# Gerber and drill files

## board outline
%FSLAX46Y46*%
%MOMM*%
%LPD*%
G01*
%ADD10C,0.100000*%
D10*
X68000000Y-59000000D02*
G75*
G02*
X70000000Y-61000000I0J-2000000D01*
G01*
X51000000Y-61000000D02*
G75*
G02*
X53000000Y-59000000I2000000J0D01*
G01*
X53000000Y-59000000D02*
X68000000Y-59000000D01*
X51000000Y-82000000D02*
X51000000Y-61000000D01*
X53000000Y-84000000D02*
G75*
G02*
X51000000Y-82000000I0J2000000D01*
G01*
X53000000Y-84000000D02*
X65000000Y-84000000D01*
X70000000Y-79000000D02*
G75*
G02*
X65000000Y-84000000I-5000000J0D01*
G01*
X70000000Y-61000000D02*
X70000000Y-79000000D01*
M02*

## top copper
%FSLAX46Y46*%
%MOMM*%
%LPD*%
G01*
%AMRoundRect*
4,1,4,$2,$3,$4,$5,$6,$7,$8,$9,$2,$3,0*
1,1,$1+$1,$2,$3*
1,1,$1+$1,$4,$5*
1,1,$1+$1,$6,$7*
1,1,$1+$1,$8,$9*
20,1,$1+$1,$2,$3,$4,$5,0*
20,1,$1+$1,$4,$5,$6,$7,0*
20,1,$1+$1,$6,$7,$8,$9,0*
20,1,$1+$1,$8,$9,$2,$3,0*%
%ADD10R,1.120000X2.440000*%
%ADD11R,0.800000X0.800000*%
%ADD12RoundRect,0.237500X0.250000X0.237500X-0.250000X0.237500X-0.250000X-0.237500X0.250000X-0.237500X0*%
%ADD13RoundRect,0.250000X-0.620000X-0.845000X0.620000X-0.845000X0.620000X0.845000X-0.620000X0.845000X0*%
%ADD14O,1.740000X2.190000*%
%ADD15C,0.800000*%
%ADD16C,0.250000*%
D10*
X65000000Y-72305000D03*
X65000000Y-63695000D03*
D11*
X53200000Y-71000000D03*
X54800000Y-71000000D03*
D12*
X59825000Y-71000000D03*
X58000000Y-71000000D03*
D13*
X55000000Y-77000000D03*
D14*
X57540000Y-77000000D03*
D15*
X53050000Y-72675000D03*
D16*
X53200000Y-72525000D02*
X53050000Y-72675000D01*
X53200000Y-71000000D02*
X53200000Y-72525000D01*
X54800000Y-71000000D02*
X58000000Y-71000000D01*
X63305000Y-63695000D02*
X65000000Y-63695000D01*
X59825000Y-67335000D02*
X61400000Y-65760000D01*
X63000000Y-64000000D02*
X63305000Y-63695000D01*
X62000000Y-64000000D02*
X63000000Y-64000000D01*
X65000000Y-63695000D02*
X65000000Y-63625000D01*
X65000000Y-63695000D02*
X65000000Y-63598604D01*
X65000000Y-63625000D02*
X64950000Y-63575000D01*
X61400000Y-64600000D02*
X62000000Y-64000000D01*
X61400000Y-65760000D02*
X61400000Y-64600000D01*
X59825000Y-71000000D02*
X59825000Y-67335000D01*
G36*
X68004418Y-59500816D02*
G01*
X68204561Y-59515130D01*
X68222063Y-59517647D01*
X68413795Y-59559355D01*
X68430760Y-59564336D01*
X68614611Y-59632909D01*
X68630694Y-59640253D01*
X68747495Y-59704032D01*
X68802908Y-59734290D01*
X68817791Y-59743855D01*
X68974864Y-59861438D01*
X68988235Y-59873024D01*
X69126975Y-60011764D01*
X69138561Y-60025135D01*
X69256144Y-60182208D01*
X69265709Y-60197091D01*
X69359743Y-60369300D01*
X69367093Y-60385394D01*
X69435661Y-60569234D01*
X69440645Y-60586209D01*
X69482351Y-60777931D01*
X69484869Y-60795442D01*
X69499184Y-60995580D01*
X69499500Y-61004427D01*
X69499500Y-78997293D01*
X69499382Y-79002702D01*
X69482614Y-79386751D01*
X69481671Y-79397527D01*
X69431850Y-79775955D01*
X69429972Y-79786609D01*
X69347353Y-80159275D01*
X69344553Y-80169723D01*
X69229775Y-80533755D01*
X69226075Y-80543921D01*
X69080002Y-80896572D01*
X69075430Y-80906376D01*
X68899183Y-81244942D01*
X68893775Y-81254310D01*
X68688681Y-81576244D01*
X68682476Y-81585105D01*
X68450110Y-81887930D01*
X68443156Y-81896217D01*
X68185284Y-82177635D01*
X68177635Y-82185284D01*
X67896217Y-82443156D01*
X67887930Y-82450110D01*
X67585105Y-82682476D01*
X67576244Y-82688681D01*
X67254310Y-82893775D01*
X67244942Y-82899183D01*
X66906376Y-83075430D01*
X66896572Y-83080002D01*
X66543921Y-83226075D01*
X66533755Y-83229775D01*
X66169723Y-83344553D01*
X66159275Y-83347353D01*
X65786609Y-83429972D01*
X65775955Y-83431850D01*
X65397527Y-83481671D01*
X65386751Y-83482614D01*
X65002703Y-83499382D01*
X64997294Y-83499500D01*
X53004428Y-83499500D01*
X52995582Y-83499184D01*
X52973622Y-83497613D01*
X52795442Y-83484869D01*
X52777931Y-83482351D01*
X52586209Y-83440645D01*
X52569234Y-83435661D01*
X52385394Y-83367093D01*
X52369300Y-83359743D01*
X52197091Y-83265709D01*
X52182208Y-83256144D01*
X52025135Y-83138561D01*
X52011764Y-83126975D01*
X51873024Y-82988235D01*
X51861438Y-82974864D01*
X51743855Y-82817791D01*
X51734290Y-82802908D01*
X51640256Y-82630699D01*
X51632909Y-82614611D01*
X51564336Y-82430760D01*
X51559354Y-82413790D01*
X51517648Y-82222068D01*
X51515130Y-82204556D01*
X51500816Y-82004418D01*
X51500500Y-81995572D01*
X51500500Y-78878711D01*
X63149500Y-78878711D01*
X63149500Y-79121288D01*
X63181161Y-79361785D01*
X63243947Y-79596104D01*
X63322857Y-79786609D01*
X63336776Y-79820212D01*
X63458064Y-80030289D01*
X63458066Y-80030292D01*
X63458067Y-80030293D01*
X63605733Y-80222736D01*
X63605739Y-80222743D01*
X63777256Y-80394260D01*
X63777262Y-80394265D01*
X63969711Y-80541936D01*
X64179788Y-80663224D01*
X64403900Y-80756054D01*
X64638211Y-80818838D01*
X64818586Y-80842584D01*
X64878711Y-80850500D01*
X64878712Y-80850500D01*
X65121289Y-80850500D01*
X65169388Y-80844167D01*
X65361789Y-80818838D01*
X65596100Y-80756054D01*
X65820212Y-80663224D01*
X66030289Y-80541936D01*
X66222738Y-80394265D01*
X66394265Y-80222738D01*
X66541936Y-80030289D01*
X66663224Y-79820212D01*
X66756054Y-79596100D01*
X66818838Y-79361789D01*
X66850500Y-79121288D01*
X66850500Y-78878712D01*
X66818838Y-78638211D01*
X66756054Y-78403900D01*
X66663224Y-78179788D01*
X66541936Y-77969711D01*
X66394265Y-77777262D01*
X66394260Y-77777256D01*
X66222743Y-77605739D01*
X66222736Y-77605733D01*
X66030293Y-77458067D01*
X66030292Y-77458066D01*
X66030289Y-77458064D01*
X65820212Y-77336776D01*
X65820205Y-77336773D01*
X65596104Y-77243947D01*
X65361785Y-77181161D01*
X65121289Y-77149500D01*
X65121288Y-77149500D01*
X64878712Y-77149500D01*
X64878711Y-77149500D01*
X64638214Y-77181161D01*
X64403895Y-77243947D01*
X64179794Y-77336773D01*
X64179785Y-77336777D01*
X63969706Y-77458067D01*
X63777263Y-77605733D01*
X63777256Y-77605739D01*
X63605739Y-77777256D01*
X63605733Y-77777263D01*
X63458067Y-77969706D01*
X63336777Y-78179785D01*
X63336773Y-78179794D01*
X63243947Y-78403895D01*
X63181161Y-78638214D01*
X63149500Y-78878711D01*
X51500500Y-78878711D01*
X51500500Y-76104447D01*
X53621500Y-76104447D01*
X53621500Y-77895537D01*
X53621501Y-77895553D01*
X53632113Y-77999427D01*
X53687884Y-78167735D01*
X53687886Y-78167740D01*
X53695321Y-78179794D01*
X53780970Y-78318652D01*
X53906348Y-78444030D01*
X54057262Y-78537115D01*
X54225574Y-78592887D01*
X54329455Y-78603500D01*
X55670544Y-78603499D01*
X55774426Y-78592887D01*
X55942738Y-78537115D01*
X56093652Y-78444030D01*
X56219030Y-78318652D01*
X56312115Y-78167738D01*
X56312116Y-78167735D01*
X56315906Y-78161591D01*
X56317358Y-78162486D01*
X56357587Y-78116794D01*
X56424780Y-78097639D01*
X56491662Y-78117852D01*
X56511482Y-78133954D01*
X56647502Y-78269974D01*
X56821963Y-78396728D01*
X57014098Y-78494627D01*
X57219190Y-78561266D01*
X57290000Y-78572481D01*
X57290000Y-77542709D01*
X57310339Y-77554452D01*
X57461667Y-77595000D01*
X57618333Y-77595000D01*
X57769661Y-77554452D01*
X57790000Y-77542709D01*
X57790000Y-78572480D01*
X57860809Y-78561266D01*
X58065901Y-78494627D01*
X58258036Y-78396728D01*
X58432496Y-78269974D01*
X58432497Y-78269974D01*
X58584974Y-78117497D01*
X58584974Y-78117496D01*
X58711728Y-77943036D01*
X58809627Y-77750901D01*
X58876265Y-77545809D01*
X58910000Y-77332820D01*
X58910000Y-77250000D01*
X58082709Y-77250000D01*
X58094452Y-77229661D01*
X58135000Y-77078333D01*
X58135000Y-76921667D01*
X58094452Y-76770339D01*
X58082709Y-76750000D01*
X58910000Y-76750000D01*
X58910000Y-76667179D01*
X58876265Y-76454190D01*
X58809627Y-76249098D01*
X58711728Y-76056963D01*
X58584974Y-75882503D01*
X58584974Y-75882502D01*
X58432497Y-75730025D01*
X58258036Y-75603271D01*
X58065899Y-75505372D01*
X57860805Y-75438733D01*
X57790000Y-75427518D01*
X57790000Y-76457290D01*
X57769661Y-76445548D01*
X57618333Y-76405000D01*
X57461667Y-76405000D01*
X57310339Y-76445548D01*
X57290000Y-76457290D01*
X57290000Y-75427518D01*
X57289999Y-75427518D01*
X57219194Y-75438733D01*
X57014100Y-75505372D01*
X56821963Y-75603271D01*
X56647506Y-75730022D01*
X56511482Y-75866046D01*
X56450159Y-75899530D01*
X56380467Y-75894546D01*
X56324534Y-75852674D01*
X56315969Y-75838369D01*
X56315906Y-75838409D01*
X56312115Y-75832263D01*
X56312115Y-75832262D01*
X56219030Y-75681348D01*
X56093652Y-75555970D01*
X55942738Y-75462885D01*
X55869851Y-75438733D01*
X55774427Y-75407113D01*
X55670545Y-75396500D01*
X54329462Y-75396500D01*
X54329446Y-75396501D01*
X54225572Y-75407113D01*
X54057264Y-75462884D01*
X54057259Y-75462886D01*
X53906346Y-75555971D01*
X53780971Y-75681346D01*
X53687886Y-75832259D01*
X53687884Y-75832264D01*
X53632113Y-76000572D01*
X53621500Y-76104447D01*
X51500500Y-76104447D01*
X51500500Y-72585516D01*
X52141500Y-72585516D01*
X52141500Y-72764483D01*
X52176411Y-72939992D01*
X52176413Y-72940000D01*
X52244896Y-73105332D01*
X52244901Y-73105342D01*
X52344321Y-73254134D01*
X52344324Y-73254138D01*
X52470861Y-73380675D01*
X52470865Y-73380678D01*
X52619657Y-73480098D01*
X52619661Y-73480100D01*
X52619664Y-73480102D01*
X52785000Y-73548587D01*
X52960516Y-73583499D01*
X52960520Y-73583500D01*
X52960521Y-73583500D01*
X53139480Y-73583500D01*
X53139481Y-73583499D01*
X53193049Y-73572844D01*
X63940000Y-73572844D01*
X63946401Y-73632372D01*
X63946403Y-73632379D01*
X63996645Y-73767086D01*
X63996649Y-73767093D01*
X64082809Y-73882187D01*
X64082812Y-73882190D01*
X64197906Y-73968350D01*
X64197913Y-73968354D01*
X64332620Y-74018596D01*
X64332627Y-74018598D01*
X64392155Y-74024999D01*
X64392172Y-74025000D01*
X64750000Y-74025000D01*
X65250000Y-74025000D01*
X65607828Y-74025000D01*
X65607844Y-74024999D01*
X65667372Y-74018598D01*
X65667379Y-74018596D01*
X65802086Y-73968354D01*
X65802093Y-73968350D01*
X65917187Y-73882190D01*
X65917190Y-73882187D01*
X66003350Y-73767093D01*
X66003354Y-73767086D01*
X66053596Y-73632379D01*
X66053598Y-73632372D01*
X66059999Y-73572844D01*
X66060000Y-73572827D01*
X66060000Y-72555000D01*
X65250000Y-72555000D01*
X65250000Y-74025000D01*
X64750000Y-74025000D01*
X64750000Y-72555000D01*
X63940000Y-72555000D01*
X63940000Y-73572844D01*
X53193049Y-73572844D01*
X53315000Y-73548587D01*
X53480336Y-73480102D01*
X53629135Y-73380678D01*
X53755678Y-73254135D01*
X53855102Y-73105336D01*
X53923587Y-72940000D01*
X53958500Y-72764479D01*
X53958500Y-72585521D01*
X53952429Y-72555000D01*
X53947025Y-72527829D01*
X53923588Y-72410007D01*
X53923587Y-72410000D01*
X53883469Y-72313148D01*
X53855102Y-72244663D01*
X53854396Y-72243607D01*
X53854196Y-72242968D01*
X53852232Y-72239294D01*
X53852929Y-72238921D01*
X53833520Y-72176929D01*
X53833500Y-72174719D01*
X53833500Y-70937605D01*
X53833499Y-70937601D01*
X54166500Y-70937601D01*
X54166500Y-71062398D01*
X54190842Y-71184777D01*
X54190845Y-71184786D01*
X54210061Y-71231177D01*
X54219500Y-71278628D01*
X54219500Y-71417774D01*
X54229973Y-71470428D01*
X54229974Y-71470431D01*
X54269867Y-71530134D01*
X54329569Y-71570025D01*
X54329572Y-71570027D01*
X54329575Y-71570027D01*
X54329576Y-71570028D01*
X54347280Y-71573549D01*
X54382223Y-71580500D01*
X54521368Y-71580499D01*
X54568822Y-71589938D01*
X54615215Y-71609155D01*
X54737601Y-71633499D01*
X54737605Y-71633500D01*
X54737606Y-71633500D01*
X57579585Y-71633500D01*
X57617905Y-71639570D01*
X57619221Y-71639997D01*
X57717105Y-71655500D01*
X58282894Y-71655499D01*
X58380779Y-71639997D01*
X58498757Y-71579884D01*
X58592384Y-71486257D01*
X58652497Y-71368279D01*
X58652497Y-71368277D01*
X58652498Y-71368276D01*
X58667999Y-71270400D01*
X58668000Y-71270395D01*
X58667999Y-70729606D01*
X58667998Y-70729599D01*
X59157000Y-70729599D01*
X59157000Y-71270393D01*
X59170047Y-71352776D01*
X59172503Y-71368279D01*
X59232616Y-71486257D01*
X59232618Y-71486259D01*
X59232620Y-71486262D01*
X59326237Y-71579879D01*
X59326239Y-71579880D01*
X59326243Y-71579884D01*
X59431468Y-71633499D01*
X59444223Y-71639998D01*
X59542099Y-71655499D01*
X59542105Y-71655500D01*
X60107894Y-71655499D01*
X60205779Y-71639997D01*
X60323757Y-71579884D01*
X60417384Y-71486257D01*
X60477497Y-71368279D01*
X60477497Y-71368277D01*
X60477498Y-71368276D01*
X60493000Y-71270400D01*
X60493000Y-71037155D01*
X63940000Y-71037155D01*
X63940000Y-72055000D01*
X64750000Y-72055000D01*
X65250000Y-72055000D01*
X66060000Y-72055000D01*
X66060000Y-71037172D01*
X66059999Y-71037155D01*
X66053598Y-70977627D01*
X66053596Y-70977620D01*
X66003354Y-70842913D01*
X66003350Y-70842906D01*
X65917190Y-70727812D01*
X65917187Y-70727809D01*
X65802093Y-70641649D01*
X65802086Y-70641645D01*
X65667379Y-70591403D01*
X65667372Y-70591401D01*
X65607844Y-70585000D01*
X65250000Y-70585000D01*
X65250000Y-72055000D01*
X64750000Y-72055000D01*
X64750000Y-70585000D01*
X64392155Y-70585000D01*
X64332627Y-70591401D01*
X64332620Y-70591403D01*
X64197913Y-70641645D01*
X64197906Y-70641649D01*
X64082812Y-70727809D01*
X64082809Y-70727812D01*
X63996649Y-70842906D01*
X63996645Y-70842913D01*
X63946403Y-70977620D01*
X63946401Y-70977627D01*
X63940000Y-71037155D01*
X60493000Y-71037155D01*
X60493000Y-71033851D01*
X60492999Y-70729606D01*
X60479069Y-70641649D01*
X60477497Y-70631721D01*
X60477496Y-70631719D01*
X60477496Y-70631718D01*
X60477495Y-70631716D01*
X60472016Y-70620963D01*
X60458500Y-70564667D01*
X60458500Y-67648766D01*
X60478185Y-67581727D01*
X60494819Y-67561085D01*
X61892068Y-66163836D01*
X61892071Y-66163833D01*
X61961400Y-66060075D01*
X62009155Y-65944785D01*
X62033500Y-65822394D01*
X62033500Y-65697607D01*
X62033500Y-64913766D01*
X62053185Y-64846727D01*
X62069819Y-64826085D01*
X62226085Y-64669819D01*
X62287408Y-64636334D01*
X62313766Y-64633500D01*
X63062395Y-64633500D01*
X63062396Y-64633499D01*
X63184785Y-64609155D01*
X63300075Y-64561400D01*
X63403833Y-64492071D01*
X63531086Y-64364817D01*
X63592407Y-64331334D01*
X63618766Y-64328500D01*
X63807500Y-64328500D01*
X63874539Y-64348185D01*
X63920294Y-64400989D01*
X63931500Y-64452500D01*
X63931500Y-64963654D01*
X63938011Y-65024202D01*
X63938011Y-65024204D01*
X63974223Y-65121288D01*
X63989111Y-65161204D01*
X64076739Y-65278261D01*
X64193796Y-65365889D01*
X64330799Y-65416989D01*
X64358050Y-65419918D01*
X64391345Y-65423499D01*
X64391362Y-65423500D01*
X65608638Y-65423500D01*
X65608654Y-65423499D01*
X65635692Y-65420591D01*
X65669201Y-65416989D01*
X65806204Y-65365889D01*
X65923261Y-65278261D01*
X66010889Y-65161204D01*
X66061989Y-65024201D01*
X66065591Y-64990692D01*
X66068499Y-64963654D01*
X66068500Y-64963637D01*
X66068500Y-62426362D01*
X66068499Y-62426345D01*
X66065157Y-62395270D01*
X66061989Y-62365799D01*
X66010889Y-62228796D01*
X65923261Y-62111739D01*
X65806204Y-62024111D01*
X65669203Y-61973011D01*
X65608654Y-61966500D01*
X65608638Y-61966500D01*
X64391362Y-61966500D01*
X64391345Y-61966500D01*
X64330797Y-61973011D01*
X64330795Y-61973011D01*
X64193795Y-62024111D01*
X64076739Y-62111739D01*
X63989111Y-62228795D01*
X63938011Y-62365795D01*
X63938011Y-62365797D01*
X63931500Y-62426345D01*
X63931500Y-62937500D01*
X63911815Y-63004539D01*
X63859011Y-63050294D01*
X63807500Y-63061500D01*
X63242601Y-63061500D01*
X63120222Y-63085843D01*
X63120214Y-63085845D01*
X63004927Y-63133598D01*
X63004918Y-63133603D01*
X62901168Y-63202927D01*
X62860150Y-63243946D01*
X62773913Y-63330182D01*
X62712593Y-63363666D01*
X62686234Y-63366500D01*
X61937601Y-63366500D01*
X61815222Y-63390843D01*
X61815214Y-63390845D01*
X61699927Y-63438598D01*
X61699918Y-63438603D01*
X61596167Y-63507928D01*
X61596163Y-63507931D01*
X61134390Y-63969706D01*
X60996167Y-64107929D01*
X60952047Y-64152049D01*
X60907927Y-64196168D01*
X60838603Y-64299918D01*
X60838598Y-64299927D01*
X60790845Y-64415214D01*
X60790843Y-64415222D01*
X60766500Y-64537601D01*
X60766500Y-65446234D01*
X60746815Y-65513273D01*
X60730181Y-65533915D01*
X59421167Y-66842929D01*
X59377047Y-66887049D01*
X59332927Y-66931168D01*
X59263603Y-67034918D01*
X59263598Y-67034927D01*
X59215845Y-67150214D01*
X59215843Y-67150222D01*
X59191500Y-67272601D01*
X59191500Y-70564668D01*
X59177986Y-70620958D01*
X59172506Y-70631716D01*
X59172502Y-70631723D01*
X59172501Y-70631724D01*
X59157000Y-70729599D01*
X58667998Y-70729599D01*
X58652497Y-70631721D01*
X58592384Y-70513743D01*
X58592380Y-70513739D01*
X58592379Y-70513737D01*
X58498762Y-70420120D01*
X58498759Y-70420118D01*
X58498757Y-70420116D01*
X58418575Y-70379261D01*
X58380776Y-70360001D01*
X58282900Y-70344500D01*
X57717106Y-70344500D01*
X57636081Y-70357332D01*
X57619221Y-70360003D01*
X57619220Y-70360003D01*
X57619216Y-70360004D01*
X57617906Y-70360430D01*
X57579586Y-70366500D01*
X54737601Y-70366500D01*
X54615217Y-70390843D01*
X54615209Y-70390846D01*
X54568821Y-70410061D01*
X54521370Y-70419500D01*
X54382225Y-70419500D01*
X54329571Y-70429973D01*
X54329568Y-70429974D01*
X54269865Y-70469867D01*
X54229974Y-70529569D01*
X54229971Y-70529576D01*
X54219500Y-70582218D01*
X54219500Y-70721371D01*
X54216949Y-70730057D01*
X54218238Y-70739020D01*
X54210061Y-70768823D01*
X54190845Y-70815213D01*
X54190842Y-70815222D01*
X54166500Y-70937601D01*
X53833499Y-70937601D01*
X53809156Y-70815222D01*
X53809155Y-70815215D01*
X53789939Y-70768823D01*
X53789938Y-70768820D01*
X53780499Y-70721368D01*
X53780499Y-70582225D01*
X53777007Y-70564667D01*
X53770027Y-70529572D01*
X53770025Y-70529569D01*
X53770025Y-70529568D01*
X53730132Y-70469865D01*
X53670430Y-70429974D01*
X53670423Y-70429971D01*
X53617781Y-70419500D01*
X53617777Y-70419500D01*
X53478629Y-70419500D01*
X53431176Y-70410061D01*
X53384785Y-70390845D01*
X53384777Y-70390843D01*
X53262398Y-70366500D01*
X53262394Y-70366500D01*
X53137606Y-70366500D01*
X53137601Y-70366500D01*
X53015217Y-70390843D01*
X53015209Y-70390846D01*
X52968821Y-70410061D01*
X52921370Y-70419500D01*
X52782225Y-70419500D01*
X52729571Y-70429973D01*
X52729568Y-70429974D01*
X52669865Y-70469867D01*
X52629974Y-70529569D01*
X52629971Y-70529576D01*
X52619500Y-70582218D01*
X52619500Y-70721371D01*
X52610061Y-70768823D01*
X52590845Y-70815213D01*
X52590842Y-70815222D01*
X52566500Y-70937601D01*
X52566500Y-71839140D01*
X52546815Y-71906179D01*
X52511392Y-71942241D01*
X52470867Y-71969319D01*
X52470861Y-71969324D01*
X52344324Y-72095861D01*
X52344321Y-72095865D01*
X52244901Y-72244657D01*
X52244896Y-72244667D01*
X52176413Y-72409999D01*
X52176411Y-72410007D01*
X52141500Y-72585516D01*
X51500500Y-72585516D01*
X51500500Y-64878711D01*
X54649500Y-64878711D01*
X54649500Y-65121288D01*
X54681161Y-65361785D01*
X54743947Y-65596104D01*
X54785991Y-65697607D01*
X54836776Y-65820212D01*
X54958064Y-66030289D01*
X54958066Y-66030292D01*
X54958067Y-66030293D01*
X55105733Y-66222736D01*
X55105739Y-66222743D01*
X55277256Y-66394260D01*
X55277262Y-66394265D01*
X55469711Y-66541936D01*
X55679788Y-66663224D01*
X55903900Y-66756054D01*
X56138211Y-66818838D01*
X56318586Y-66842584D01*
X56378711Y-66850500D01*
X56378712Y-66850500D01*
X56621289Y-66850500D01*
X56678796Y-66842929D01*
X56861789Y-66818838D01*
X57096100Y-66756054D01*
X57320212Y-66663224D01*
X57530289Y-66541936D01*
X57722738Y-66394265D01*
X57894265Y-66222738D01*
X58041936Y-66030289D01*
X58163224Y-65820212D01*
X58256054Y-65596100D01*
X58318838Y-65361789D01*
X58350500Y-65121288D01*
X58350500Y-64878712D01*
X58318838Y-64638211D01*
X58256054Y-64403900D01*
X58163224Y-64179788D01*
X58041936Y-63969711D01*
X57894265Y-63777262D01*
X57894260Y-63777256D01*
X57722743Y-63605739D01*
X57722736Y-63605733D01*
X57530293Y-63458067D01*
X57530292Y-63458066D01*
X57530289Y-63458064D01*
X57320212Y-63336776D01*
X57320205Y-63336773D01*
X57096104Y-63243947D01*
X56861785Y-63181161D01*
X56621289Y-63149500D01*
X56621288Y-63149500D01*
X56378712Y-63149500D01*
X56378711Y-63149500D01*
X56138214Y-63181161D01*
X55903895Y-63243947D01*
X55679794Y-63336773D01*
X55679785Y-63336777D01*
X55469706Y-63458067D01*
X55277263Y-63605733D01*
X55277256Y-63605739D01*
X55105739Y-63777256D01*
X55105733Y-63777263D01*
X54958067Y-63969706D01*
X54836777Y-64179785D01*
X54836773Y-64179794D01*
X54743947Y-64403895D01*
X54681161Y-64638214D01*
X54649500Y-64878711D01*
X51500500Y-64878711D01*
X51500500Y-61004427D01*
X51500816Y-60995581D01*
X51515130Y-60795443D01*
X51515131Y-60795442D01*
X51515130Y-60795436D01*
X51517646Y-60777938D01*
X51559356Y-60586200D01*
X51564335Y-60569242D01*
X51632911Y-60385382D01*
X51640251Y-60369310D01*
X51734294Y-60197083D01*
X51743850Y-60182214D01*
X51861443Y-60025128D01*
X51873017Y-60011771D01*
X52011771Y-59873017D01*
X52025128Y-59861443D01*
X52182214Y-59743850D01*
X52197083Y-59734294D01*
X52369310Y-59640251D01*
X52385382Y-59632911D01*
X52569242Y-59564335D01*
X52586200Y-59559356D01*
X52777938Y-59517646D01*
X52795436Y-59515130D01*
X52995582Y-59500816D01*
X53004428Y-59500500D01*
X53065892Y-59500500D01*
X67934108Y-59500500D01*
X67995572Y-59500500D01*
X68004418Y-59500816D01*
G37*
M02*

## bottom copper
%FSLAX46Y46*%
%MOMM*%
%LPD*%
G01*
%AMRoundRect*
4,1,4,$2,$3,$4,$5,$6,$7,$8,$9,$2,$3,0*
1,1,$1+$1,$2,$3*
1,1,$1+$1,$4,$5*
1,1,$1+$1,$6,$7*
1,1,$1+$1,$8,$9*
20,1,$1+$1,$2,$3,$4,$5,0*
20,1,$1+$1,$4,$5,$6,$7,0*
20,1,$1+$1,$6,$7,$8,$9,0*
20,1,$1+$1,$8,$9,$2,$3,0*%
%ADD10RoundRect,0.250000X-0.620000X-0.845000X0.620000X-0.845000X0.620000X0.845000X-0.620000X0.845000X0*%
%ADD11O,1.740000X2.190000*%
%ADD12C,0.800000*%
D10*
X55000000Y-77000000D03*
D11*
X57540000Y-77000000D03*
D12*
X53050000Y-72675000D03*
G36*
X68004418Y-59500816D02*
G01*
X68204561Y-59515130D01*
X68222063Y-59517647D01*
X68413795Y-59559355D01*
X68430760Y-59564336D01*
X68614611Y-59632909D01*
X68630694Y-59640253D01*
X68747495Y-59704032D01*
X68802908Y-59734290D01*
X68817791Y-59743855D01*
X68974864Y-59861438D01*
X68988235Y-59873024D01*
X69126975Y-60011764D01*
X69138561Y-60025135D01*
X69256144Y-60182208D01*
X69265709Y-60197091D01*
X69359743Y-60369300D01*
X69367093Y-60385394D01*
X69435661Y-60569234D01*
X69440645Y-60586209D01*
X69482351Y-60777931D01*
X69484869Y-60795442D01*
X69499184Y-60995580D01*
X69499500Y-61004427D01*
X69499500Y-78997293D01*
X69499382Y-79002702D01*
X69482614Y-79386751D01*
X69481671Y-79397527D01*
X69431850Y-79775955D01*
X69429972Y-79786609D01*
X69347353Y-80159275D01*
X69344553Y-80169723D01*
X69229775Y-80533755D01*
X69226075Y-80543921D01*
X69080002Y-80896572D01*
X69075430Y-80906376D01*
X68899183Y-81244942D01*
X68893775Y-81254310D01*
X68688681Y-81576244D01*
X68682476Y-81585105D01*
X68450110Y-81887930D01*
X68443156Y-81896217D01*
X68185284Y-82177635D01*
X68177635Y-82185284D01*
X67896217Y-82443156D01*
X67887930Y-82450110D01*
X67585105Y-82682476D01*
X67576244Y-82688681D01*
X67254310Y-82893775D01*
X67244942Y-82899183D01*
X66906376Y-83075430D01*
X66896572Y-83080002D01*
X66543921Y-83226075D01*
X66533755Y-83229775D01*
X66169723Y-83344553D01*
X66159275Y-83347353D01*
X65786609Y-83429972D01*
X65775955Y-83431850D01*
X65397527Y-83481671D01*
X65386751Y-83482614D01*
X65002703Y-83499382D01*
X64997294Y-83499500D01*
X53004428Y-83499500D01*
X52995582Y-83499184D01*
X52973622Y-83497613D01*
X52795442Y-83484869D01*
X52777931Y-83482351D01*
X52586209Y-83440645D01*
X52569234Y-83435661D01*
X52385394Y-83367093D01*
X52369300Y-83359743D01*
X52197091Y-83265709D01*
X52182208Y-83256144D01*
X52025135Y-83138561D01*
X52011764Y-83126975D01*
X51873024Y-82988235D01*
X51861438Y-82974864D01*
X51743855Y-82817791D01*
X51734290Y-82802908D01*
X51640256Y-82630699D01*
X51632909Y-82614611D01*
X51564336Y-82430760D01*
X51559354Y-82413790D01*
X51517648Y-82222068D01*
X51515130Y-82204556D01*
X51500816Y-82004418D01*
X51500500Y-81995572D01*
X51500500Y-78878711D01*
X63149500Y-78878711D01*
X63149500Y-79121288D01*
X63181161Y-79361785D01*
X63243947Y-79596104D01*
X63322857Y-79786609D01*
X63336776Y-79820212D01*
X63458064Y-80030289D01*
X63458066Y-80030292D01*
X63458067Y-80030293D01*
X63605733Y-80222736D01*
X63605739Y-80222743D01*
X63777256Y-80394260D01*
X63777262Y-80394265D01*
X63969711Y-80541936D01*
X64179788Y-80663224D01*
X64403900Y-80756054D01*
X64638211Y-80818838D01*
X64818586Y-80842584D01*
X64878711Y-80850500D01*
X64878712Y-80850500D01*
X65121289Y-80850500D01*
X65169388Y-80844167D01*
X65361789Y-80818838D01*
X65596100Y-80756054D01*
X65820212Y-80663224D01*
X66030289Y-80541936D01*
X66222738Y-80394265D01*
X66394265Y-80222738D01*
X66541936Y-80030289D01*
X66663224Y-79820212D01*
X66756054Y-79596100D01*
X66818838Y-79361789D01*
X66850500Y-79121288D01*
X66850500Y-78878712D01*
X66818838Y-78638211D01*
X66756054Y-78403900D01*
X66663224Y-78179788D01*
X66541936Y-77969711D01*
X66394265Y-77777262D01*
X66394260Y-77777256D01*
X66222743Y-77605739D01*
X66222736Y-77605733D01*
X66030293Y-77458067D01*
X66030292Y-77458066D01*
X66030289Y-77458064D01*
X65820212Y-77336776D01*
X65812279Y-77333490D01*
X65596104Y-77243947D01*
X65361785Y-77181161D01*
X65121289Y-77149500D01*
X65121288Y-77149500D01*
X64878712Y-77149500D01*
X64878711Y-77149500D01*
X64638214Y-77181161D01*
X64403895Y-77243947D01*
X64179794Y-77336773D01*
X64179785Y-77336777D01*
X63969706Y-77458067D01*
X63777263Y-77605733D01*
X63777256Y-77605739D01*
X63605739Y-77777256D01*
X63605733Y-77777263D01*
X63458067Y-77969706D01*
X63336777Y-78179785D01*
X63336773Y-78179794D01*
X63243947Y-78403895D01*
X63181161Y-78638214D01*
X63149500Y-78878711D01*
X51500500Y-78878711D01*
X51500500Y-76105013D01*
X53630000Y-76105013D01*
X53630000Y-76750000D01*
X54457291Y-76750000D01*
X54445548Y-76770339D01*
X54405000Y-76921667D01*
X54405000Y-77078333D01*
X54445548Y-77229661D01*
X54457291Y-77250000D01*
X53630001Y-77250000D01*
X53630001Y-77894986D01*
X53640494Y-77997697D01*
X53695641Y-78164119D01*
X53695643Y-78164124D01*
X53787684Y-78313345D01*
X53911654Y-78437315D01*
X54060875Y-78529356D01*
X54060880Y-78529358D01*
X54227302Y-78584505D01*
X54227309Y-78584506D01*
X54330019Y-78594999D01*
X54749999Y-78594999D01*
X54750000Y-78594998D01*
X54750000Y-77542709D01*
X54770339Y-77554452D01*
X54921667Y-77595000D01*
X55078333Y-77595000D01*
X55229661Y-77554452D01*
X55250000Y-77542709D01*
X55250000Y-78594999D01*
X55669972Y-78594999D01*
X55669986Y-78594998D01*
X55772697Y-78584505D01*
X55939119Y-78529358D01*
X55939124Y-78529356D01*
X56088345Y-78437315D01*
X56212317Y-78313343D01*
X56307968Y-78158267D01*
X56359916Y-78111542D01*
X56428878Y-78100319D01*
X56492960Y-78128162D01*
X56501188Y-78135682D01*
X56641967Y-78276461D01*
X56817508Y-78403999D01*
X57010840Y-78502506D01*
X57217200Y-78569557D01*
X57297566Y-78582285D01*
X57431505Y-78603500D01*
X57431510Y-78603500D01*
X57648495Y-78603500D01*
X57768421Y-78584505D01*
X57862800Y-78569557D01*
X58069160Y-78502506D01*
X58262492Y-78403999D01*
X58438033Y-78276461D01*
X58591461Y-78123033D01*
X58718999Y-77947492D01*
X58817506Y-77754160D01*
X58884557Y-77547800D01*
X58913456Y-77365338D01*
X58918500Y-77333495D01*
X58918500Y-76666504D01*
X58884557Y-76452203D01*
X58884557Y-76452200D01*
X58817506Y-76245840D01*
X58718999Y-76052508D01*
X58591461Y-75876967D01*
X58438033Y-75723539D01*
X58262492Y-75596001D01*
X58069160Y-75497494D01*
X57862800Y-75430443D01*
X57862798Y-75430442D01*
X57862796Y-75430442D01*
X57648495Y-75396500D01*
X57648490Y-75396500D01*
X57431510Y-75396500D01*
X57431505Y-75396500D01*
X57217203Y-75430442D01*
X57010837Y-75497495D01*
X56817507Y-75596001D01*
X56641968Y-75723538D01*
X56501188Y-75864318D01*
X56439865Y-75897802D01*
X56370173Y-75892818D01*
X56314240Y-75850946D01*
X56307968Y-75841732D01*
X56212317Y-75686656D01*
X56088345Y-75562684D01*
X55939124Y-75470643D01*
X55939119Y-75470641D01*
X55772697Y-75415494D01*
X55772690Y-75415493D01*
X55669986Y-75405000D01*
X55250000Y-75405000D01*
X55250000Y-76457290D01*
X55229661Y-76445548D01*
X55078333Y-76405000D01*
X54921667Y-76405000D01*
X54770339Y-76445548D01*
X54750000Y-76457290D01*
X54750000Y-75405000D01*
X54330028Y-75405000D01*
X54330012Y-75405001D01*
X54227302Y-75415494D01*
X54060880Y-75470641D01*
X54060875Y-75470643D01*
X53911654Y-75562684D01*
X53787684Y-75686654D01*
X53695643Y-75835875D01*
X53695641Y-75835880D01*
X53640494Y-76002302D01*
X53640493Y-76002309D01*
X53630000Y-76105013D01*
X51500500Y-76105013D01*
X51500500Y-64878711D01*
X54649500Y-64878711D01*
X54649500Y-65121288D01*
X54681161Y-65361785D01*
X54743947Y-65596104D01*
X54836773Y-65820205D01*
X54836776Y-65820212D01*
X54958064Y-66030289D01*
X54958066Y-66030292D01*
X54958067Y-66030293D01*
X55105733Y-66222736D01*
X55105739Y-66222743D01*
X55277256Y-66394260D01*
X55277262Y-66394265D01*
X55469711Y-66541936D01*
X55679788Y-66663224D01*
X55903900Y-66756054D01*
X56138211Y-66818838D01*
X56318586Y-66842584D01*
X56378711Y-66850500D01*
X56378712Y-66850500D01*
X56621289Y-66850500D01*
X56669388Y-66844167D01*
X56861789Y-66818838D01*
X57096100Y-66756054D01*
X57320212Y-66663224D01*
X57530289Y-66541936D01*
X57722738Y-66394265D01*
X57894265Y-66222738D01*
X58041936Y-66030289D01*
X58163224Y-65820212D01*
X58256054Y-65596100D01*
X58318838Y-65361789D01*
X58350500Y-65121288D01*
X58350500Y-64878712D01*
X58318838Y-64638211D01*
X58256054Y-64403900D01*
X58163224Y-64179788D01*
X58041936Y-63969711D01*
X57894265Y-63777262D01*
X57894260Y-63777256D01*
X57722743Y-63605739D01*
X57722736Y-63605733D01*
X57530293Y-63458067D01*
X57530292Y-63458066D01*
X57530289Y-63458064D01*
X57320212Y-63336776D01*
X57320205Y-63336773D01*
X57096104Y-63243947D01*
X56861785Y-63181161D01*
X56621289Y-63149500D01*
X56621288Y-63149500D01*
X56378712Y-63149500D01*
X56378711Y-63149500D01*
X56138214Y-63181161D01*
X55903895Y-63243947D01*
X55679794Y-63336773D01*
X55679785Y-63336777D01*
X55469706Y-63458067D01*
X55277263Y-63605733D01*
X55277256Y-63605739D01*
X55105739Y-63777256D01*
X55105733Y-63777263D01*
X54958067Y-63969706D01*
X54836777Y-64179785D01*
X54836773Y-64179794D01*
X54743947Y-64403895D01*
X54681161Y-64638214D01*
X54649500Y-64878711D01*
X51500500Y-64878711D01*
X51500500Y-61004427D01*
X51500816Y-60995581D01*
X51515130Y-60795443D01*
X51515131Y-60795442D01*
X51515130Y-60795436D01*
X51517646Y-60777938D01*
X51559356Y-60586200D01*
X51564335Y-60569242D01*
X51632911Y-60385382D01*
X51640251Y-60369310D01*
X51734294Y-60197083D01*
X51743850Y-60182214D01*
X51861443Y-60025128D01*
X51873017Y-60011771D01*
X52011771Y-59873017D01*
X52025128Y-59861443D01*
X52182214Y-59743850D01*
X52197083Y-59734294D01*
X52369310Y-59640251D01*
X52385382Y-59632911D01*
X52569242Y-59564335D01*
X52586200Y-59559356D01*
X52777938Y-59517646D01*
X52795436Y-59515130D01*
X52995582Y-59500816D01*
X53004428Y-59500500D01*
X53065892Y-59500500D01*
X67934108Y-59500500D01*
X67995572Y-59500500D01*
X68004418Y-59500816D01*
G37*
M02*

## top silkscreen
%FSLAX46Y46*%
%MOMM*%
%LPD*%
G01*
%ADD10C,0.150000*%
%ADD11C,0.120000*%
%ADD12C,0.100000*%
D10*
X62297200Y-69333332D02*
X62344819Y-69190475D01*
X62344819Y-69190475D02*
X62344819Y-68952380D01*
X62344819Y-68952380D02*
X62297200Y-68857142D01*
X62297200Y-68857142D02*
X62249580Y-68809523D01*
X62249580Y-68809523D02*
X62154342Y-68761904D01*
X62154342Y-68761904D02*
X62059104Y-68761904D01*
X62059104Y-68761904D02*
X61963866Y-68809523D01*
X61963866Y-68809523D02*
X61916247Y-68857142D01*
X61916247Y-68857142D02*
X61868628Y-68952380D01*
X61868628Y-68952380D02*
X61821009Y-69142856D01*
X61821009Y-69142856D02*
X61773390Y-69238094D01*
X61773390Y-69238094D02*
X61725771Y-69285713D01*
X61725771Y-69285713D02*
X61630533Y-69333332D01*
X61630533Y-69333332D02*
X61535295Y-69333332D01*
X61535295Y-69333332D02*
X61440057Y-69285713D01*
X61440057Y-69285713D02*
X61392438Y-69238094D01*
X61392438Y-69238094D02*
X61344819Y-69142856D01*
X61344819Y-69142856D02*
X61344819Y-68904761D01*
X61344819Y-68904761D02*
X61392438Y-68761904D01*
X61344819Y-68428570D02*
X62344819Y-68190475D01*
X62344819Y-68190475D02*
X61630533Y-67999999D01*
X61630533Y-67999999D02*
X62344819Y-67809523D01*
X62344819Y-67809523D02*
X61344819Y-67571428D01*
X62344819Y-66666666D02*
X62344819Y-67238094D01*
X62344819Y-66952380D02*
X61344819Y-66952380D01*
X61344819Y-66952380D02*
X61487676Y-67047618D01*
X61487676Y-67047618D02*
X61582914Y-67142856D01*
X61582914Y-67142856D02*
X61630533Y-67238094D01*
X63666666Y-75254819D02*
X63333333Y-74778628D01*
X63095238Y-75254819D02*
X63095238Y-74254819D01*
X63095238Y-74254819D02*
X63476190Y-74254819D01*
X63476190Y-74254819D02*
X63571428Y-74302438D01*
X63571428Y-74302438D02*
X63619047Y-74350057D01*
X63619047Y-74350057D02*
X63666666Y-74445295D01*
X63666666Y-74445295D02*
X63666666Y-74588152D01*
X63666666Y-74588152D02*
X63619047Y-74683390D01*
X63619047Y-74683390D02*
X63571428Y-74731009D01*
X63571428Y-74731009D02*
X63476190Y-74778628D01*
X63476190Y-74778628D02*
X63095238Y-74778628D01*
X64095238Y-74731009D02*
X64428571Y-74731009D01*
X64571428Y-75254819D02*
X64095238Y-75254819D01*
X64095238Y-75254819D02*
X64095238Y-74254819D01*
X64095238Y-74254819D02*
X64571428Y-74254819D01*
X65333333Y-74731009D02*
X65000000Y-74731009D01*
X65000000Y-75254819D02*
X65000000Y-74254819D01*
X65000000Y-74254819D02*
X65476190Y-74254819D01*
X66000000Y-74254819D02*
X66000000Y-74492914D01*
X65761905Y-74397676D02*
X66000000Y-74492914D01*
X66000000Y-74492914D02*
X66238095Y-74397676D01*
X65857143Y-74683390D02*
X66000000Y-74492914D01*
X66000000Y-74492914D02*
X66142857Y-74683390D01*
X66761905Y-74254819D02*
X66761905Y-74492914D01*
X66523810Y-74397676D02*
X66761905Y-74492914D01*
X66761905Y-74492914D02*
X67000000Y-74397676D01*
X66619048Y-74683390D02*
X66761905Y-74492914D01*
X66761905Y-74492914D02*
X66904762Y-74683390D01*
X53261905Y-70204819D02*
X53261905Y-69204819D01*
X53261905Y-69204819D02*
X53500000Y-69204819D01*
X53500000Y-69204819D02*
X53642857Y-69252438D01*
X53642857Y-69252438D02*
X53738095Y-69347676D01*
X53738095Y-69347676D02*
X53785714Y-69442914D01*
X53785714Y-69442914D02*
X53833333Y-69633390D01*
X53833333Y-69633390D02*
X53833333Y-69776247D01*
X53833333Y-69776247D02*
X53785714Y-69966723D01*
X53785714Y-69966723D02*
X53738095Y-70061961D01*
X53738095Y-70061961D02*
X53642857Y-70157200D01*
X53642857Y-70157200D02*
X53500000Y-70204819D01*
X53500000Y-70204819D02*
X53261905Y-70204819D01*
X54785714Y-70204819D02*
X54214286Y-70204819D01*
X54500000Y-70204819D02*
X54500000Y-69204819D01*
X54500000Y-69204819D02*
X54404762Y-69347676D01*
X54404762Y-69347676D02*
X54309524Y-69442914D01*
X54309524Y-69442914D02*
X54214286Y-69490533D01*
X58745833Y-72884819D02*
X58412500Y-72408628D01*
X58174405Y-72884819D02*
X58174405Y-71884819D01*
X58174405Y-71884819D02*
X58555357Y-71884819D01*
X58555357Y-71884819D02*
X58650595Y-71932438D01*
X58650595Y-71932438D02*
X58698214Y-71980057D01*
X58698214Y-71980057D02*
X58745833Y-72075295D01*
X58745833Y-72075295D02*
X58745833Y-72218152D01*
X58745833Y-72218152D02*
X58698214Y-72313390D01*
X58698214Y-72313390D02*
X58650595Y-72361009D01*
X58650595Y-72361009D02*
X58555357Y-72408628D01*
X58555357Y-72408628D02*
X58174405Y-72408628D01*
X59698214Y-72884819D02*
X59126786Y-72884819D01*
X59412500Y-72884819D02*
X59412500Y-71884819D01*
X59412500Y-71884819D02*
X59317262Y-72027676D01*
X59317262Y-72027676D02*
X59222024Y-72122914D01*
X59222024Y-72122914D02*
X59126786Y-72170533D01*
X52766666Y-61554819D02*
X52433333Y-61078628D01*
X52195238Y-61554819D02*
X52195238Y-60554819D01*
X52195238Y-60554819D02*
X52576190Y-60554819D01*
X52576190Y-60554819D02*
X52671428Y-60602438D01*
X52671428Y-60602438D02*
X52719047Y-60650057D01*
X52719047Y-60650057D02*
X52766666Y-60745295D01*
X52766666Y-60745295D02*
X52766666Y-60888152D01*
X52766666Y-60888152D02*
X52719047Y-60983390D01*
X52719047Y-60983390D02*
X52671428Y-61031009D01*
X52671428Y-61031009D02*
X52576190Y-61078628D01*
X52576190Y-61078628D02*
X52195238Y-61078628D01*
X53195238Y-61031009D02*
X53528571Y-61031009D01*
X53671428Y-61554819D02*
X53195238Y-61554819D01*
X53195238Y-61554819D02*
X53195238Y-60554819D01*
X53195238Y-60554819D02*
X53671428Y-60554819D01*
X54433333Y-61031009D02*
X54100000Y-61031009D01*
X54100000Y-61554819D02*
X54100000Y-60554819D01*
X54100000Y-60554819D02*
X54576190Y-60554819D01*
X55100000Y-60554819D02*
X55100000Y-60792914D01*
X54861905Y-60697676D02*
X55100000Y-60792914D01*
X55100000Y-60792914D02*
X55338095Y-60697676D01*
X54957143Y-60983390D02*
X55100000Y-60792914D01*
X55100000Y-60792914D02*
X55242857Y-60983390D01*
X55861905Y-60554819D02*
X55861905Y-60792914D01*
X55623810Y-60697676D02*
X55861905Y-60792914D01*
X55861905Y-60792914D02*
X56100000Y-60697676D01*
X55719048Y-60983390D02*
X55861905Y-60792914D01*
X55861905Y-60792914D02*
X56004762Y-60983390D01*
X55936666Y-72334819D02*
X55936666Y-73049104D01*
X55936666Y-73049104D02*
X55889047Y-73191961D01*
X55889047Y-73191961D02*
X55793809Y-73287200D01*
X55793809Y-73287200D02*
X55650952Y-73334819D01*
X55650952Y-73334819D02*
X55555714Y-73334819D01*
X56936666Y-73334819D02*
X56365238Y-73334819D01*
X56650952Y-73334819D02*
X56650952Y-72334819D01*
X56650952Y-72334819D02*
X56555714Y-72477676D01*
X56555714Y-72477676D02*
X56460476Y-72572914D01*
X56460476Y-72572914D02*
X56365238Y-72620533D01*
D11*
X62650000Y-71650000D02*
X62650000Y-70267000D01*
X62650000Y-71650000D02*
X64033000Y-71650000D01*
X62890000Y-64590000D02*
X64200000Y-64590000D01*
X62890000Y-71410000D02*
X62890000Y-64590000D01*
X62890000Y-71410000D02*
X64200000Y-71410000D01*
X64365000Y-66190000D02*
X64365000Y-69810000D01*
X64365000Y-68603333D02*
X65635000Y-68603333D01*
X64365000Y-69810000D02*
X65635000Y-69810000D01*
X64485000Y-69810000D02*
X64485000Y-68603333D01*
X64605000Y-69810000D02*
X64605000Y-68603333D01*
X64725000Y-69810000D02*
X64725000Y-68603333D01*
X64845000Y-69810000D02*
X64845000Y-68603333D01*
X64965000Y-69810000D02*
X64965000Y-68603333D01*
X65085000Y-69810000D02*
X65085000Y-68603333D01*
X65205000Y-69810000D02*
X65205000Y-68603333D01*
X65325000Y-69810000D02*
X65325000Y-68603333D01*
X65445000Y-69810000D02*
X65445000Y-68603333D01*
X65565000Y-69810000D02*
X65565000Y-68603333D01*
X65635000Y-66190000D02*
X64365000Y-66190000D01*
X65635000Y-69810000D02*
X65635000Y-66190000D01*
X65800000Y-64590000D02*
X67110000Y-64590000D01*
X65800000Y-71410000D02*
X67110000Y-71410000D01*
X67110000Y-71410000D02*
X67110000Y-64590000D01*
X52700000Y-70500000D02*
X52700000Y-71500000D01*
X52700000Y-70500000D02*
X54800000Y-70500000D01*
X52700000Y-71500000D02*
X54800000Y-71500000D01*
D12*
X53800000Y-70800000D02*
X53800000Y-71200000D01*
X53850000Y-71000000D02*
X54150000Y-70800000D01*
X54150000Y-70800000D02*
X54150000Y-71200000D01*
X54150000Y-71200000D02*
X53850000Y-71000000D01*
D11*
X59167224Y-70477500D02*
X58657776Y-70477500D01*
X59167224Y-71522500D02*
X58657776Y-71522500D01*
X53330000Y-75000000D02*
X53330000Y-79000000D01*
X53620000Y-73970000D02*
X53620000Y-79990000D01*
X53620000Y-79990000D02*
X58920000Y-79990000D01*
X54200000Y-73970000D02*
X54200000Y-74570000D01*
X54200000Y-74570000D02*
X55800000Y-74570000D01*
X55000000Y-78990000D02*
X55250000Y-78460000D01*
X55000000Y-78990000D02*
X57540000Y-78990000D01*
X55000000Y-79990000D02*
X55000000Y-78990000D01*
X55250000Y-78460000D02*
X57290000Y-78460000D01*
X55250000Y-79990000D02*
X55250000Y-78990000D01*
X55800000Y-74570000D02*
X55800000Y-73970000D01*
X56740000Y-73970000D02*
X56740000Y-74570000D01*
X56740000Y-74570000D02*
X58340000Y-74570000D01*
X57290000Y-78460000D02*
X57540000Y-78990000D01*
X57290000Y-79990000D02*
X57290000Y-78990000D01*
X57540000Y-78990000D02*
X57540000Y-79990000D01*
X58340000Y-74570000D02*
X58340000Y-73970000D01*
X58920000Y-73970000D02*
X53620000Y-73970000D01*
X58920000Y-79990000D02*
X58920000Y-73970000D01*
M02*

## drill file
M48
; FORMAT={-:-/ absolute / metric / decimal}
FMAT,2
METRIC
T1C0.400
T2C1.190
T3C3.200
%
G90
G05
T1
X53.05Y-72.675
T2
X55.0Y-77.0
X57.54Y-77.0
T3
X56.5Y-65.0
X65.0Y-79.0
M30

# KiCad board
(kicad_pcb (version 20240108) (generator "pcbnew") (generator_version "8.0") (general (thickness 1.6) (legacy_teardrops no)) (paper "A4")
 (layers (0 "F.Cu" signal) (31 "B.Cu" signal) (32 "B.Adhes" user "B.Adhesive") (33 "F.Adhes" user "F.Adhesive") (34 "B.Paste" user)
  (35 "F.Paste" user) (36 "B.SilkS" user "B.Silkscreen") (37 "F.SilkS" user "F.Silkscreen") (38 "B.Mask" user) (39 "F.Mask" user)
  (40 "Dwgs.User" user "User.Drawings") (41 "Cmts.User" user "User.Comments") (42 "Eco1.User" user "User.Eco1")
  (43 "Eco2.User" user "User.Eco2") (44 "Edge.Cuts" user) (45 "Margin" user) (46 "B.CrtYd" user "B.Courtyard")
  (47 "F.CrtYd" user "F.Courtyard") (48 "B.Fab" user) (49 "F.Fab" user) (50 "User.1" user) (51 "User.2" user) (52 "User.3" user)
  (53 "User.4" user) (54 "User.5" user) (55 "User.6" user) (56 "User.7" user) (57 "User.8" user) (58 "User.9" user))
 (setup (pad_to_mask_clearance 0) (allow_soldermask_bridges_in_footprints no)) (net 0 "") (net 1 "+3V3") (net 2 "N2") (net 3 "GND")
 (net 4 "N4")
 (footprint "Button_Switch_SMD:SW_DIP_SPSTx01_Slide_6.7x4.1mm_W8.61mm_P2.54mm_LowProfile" (layer "F.Cu") (at 65 68 90)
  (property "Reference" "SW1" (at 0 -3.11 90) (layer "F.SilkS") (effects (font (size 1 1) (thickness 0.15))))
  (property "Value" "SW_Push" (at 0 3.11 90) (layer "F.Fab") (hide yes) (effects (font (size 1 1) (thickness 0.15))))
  (fp_line (start -3.65 -2.35) (end -2.267 -2.35) (stroke (width 0.12) (type solid)) (layer "F.SilkS"))
  (fp_line (start -3.65 -2.35) (end -3.65 -0.967) (stroke (width 0.12) (type solid)) (layer "F.SilkS"))
  (fp_line (start 3.41 -2.11) (end 3.41 -0.8) (stroke (width 0.12) (type solid)) (layer "F.SilkS"))
  (fp_line (start -3.41 -2.11) (end 3.41 -2.11) (stroke (width 0.12) (type solid)) (layer "F.SilkS"))
  (fp_line (start -3.41 -2.11) (end -3.41 -0.8) (stroke (width 0.12) (type solid)) (layer "F.SilkS"))
  (fp_line (start 1.81 -0.635) (end -1.81 -0.635) (stroke (width 0.12) (type solid)) (layer "F.SilkS"))
  (fp_line (start -0.603333 -0.635) (end -0.603333 0.635) (stroke (width 0.12) (type solid)) (layer "F.SilkS"))
  (fp_line (start -1.81 -0.635) (end -1.81 0.635) (stroke (width 0.12) (type solid)) (layer "F.SilkS"))
  (fp_line (start -1.81 -0.515) (end -0.603333 -0.515) (stroke (width 0.12) (type solid)) (layer "F.SilkS"))
  (fp_line (start -1.81 -0.395) (end -0.603333 -0.395) (stroke (width 0.12) (type solid)) (layer "F.SilkS"))
  (fp_line (start -1.81 -0.275) (end -0.603333 -0.275) (stroke (width 0.12) (type solid)) (layer "F.SilkS"))
  (fp_line (start -1.81 -0.155) (end -0.603333 -0.155) (stroke (width 0.12) (type solid)) (layer "F.SilkS"))
  (fp_line (start -1.81 -0.035) (end -0.603333 -0.035) (stroke (width 0.12) (type solid)) (layer "F.SilkS"))
  (fp_line (start -1.81 0.085) (end -0.603333 0.085) (stroke (width 0.12) (type solid)) (layer "F.SilkS"))
  (fp_line (start -1.81 0.205) (end -0.603333 0.205) (stroke (width 0.12) (type solid)) (layer "F.SilkS"))
  (fp_line (start -1.81 0.325) (end -0.603333 0.325) (stroke (width 0.12) (type solid)) (layer "F.SilkS"))
  (fp_line (start -1.81 0.445) (end -0.603333 0.445) (stroke (width 0.12) (type solid)) (layer "F.SilkS"))
  (fp_line (start -1.81 0.565) (end -0.603333 0.565) (stroke (width 0.12) (type solid)) (layer "F.SilkS"))
  (fp_line (start 1.81 0.635) (end 1.81 -0.635) (stroke (width 0.12) (type solid)) (layer "F.SilkS"))
  (fp_line (start -1.81 0.635) (end 1.81 0.635) (stroke (width 0.12) (type solid)) (layer "F.SilkS"))
  (fp_line (start 3.41 0.8) (end 3.41 2.11) (stroke (width 0.12) (type solid)) (layer "F.SilkS"))
  (fp_line (start -3.41 0.8) (end -3.41 2.11) (stroke (width 0.12) (type solid)) (layer "F.SilkS"))
  (fp_line (start -3.41 2.11) (end 3.41 2.11) (stroke (width 0.12) (type solid)) (layer "F.SilkS"))
  (pad "1" smd rect (at -4.305 0 90) (size 2.44 1.12) (layers "F.Cu" "F.Paste" "F.Mask") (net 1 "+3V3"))
  (pad "2" smd rect (at 4.305 0 90) (size 2.44 1.12) (layers "F.Cu" "F.Paste" "F.Mask") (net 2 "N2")))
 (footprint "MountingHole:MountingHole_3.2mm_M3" (layer "F.Cu") (at 65 79)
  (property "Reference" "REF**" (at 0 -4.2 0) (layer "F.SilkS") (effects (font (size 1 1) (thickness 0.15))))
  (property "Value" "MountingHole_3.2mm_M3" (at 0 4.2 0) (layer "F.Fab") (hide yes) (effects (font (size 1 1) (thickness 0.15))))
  (pad "" np_thru_hole circle (at 0 0) (size 3.2 3.2) (drill 3.2) (layers "F&B.Cu" "*.Mask")))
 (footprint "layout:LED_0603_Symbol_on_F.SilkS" (layer "F.Cu") (at 54 71)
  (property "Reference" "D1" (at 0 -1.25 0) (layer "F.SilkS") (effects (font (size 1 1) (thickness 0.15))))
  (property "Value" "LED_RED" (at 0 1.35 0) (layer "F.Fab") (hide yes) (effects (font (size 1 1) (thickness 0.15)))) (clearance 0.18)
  (fp_line (start -1.3 -0.5) (end -1.3 0.5) (stroke (width 0.12) (type solid)) (layer "F.SilkS"))
  (fp_line (start -1.3 -0.5) (end 0.8 -0.5) (stroke (width 0.12) (type solid)) (layer "F.SilkS"))
  (fp_line (start -1.3 0.5) (end 0.8 0.5) (stroke (width 0.12) (type solid)) (layer "F.SilkS"))
  (fp_line (start -0.2 -0.2) (end -0.2 0.2) (stroke (width 0.1) (type solid)) (layer "F.SilkS"))
  (fp_line (start -0.15 0) (end 0.15 -0.2) (stroke (width 0.1) (type solid)) (layer "F.SilkS"))
  (fp_line (start 0.15 -0.2) (end 0.15 0.2) (stroke (width 0.1) (type solid)) (layer "F.SilkS"))
  (fp_line (start 0.15 0.2) (end -0.15 0) (stroke (width 0.1) (type solid)) (layer "F.SilkS"))
  (pad "1" smd rect (at -0.8 0 180) (size 0.8 0.8) (layers "F.Cu" "F.Paste" "F.Mask") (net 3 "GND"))
  (pad "2" smd rect (at 0.8 0 180) (size 0.8 0.8) (layers "F.Cu" "F.Paste" "F.Mask") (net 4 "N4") (clearance 0.18)))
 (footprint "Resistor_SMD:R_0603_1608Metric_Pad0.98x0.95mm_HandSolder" (layer "F.Cu") (at 58.9125 71 180)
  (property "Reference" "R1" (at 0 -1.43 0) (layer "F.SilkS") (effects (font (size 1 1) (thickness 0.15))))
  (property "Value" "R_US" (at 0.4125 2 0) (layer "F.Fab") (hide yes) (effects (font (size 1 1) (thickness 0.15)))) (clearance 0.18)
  (fp_line (start -0.254724 0.5225) (end 0.254724 0.5225) (stroke (width 0.12) (type solid)) (layer "F.SilkS"))
  (fp_line (start -0.254724 -0.5225) (end 0.254724 -0.5225) (stroke (width 0.12) (type solid)) (layer "F.SilkS"))
  (pad "1" smd roundrect (at -0.9125 0 180) (size 0.975 0.95) (layers "F.Cu" "F.Paste" "F.Mask") (roundrect_rratio 0.25) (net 2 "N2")
   (clearance 0.18))
  (pad "2" smd roundrect (at 0.9125 0 180) (size 0.975 0.95) (layers "F.Cu" "F.Paste" "F.Mask") (roundrect_rratio 0.25) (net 4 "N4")))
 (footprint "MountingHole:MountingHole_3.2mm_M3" (layer "F.Cu") (at 56.5 65)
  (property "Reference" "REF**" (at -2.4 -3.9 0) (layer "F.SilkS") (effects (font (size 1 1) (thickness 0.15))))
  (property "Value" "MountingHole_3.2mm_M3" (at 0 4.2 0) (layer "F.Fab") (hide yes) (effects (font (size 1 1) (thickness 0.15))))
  (pad "" np_thru_hole circle (at 0 0) (size 3.2 3.2) (drill 3.2) (layers "*.Cu" "*.Mask")))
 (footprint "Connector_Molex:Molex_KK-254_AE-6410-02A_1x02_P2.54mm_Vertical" (layer "F.Cu") (at 55 77)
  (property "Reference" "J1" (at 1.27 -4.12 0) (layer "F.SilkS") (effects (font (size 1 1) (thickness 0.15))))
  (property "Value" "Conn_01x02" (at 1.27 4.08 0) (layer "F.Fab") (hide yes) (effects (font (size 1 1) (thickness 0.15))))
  (fp_line (start -1.67 -2) (end -1.67 2) (stroke (width 0.12) (type solid)) (layer "F.SilkS"))
  (fp_line (start -1.38 -3.03) (end -1.38 2.99) (stroke (width 0.12) (type solid)) (layer "F.SilkS"))
  (fp_line (start -1.38 2.99) (end 3.92 2.99) (stroke (width 0.12) (type solid)) (layer "F.SilkS"))
  (fp_line (start -0.8 -3.03) (end -0.8 -2.43) (stroke (width 0.12) (type solid)) (layer "F.SilkS"))
  (fp_line (start -0.8 -2.43) (end 0.8 -2.43) (stroke (width 0.12) (type solid)) (layer "F.SilkS"))
  (fp_line (start 0 1.99) (end 0.25 1.46) (stroke (width 0.12) (type solid)) (layer "F.SilkS"))
  (fp_line (start 0 1.99) (end 2.54 1.99) (stroke (width 0.12) (type solid)) (layer "F.SilkS"))
  (fp_line (start 0 2.99) (end 0 1.99) (stroke (width 0.12) (type solid)) (layer "F.SilkS"))
  (fp_line (start 0.25 1.46) (end 2.29 1.46) (stroke (width 0.12) (type solid)) (layer "F.SilkS"))
  (fp_line (start 0.25 2.99) (end 0.25 1.99) (stroke (width 0.12) (type solid)) (layer "F.SilkS"))
  (fp_line (start 0.8 -2.43) (end 0.8 -3.03) (stroke (width 0.12) (type solid)) (layer "F.SilkS"))
  (fp_line (start 1.74 -3.03) (end 1.74 -2.43) (stroke (width 0.12) (type solid)) (layer "F.SilkS"))
  (fp_line (start 1.74 -2.43) (end 3.34 -2.43) (stroke (width 0.12) (type solid)) (layer "F.SilkS"))
  (fp_line (start 2.29 1.46) (end 2.54 1.99) (stroke (width 0.12) (type solid)) (layer "F.SilkS"))
  (fp_line (start 2.29 2.99) (end 2.29 1.99) (stroke (width 0.12) (type solid)) (layer "F.SilkS"))
  (fp_line (start 2.54 1.99) (end 2.54 2.99) (stroke (width 0.12) (type solid)) (layer "F.SilkS"))
  (fp_line (start 3.34 -2.43) (end 3.34 -3.03) (stroke (width 0.12) (type solid)) (layer "F.SilkS"))
  (fp_line (start 3.92 -3.03) (end -1.38 -3.03) (stroke (width 0.12) (type solid)) (layer "F.SilkS"))
  (fp_line (start 3.92 2.99) (end 3.92 -3.03) (stroke (width 0.12) (type solid)) (layer "F.SilkS"))
  (pad "1" thru_hole roundrect (at 0 0) (size 1.74 2.19) (drill 1.19) (layers "*.Cu" "*.Mask") (remove_unused_layers no)
   (roundrect_rratio 0.143678) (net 3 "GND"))
  (pad "2" thru_hole oval (at 2.54 0) (size 1.74 2.19) (drill 1.19) (layers "*.Cu" "*.Mask") (remove_unused_layers no) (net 1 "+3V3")))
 (gr_arc (start 68 59) (mid 69.414214 59.585786) (end 70 61) (stroke (width 0.1) (type default)) (layer "Edge.Cuts"))
 (gr_arc (start 51 61) (mid 51.585786 59.585786) (end 53 59) (stroke (width 0.1) (type default)) (layer "Edge.Cuts"))
 (gr_line (start 53 59) (end 68 59) (stroke (width 0.1) (type default)) (layer "Edge.Cuts"))
 (gr_line (start 51 82) (end 51 61) (stroke (width 0.1) (type default)) (layer "Edge.Cuts"))
 (gr_arc (start 53 84) (mid 51.585786 83.414214) (end 51 82) (stroke (width 0.1) (type default)) (layer "Edge.Cuts"))
 (gr_line (start 53 84) (end 65 84) (stroke (width 0.1) (type default)) (layer "Edge.Cuts"))
 (gr_arc (start 70 79) (mid 68.535534 82.535534) (end 65 84) (stroke (width 0.1) (type default)) (layer "Edge.Cuts"))
 (gr_line (start 70 61) (end 70 79) (stroke (width 0.1) (type default)) (layer "Edge.Cuts"))
 (segment (start 53.2 72.525) (end 53.05 72.675) (width 0.25) (layer "F.Cu") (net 3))
 (segment (start 53.2 71) (end 53.2 72.525) (width 0.25) (layer "F.Cu") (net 3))
 (via (at 53.05 72.675) (size 0.8) (drill 0.4) (layers "F.Cu" "B.Cu") (free yes) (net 3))
 (segment (start 54.8 71) (end 58 71) (width 0.25) (layer "F.Cu") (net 4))
 (segment (start 63.305 63.695) (end 65 63.695) (width 0.25) (layer "F.Cu") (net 2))
 (segment (start 59.825 67.335) (end 61.4 65.76) (width 0.25) (layer "F.Cu") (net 2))
 (segment (start 63 64) (end 63.305 63.695) (width 0.25) (layer "F.Cu") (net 2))
 (segment (start 62 64) (end 63 64) (width 0.25) (layer "F.Cu") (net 2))
 (segment (start 65 63.695) (end 65 63.625) (width 0.25) (layer "F.Cu") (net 2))
 (segment (start 65 63.695) (end 65 63.598604) (width 0.25) (layer "F.Cu") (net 2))
 (segment (start 65 63.625) (end 64.95 63.575) (width 0.25) (layer "F.Cu") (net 2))
 (segment (start 61.4 64.6) (end 62 64) (width 0.25) (layer "F.Cu") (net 2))
 (segment (start 61.4 65.76) (end 61.4 64.6) (width 0.25) (layer "F.Cu") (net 2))
 (segment (start 59.825 71) (end 59.825 67.335) (width 0.25) (layer "F.Cu") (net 2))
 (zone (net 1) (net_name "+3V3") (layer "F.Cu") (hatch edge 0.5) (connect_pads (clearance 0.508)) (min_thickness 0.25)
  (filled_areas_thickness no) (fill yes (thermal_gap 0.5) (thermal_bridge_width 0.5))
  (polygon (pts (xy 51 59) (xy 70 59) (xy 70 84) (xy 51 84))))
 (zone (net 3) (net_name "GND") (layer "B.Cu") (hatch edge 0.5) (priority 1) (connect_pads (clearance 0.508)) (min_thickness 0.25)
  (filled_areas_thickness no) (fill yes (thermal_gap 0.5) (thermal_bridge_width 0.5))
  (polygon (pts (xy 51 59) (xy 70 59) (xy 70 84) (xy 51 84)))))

